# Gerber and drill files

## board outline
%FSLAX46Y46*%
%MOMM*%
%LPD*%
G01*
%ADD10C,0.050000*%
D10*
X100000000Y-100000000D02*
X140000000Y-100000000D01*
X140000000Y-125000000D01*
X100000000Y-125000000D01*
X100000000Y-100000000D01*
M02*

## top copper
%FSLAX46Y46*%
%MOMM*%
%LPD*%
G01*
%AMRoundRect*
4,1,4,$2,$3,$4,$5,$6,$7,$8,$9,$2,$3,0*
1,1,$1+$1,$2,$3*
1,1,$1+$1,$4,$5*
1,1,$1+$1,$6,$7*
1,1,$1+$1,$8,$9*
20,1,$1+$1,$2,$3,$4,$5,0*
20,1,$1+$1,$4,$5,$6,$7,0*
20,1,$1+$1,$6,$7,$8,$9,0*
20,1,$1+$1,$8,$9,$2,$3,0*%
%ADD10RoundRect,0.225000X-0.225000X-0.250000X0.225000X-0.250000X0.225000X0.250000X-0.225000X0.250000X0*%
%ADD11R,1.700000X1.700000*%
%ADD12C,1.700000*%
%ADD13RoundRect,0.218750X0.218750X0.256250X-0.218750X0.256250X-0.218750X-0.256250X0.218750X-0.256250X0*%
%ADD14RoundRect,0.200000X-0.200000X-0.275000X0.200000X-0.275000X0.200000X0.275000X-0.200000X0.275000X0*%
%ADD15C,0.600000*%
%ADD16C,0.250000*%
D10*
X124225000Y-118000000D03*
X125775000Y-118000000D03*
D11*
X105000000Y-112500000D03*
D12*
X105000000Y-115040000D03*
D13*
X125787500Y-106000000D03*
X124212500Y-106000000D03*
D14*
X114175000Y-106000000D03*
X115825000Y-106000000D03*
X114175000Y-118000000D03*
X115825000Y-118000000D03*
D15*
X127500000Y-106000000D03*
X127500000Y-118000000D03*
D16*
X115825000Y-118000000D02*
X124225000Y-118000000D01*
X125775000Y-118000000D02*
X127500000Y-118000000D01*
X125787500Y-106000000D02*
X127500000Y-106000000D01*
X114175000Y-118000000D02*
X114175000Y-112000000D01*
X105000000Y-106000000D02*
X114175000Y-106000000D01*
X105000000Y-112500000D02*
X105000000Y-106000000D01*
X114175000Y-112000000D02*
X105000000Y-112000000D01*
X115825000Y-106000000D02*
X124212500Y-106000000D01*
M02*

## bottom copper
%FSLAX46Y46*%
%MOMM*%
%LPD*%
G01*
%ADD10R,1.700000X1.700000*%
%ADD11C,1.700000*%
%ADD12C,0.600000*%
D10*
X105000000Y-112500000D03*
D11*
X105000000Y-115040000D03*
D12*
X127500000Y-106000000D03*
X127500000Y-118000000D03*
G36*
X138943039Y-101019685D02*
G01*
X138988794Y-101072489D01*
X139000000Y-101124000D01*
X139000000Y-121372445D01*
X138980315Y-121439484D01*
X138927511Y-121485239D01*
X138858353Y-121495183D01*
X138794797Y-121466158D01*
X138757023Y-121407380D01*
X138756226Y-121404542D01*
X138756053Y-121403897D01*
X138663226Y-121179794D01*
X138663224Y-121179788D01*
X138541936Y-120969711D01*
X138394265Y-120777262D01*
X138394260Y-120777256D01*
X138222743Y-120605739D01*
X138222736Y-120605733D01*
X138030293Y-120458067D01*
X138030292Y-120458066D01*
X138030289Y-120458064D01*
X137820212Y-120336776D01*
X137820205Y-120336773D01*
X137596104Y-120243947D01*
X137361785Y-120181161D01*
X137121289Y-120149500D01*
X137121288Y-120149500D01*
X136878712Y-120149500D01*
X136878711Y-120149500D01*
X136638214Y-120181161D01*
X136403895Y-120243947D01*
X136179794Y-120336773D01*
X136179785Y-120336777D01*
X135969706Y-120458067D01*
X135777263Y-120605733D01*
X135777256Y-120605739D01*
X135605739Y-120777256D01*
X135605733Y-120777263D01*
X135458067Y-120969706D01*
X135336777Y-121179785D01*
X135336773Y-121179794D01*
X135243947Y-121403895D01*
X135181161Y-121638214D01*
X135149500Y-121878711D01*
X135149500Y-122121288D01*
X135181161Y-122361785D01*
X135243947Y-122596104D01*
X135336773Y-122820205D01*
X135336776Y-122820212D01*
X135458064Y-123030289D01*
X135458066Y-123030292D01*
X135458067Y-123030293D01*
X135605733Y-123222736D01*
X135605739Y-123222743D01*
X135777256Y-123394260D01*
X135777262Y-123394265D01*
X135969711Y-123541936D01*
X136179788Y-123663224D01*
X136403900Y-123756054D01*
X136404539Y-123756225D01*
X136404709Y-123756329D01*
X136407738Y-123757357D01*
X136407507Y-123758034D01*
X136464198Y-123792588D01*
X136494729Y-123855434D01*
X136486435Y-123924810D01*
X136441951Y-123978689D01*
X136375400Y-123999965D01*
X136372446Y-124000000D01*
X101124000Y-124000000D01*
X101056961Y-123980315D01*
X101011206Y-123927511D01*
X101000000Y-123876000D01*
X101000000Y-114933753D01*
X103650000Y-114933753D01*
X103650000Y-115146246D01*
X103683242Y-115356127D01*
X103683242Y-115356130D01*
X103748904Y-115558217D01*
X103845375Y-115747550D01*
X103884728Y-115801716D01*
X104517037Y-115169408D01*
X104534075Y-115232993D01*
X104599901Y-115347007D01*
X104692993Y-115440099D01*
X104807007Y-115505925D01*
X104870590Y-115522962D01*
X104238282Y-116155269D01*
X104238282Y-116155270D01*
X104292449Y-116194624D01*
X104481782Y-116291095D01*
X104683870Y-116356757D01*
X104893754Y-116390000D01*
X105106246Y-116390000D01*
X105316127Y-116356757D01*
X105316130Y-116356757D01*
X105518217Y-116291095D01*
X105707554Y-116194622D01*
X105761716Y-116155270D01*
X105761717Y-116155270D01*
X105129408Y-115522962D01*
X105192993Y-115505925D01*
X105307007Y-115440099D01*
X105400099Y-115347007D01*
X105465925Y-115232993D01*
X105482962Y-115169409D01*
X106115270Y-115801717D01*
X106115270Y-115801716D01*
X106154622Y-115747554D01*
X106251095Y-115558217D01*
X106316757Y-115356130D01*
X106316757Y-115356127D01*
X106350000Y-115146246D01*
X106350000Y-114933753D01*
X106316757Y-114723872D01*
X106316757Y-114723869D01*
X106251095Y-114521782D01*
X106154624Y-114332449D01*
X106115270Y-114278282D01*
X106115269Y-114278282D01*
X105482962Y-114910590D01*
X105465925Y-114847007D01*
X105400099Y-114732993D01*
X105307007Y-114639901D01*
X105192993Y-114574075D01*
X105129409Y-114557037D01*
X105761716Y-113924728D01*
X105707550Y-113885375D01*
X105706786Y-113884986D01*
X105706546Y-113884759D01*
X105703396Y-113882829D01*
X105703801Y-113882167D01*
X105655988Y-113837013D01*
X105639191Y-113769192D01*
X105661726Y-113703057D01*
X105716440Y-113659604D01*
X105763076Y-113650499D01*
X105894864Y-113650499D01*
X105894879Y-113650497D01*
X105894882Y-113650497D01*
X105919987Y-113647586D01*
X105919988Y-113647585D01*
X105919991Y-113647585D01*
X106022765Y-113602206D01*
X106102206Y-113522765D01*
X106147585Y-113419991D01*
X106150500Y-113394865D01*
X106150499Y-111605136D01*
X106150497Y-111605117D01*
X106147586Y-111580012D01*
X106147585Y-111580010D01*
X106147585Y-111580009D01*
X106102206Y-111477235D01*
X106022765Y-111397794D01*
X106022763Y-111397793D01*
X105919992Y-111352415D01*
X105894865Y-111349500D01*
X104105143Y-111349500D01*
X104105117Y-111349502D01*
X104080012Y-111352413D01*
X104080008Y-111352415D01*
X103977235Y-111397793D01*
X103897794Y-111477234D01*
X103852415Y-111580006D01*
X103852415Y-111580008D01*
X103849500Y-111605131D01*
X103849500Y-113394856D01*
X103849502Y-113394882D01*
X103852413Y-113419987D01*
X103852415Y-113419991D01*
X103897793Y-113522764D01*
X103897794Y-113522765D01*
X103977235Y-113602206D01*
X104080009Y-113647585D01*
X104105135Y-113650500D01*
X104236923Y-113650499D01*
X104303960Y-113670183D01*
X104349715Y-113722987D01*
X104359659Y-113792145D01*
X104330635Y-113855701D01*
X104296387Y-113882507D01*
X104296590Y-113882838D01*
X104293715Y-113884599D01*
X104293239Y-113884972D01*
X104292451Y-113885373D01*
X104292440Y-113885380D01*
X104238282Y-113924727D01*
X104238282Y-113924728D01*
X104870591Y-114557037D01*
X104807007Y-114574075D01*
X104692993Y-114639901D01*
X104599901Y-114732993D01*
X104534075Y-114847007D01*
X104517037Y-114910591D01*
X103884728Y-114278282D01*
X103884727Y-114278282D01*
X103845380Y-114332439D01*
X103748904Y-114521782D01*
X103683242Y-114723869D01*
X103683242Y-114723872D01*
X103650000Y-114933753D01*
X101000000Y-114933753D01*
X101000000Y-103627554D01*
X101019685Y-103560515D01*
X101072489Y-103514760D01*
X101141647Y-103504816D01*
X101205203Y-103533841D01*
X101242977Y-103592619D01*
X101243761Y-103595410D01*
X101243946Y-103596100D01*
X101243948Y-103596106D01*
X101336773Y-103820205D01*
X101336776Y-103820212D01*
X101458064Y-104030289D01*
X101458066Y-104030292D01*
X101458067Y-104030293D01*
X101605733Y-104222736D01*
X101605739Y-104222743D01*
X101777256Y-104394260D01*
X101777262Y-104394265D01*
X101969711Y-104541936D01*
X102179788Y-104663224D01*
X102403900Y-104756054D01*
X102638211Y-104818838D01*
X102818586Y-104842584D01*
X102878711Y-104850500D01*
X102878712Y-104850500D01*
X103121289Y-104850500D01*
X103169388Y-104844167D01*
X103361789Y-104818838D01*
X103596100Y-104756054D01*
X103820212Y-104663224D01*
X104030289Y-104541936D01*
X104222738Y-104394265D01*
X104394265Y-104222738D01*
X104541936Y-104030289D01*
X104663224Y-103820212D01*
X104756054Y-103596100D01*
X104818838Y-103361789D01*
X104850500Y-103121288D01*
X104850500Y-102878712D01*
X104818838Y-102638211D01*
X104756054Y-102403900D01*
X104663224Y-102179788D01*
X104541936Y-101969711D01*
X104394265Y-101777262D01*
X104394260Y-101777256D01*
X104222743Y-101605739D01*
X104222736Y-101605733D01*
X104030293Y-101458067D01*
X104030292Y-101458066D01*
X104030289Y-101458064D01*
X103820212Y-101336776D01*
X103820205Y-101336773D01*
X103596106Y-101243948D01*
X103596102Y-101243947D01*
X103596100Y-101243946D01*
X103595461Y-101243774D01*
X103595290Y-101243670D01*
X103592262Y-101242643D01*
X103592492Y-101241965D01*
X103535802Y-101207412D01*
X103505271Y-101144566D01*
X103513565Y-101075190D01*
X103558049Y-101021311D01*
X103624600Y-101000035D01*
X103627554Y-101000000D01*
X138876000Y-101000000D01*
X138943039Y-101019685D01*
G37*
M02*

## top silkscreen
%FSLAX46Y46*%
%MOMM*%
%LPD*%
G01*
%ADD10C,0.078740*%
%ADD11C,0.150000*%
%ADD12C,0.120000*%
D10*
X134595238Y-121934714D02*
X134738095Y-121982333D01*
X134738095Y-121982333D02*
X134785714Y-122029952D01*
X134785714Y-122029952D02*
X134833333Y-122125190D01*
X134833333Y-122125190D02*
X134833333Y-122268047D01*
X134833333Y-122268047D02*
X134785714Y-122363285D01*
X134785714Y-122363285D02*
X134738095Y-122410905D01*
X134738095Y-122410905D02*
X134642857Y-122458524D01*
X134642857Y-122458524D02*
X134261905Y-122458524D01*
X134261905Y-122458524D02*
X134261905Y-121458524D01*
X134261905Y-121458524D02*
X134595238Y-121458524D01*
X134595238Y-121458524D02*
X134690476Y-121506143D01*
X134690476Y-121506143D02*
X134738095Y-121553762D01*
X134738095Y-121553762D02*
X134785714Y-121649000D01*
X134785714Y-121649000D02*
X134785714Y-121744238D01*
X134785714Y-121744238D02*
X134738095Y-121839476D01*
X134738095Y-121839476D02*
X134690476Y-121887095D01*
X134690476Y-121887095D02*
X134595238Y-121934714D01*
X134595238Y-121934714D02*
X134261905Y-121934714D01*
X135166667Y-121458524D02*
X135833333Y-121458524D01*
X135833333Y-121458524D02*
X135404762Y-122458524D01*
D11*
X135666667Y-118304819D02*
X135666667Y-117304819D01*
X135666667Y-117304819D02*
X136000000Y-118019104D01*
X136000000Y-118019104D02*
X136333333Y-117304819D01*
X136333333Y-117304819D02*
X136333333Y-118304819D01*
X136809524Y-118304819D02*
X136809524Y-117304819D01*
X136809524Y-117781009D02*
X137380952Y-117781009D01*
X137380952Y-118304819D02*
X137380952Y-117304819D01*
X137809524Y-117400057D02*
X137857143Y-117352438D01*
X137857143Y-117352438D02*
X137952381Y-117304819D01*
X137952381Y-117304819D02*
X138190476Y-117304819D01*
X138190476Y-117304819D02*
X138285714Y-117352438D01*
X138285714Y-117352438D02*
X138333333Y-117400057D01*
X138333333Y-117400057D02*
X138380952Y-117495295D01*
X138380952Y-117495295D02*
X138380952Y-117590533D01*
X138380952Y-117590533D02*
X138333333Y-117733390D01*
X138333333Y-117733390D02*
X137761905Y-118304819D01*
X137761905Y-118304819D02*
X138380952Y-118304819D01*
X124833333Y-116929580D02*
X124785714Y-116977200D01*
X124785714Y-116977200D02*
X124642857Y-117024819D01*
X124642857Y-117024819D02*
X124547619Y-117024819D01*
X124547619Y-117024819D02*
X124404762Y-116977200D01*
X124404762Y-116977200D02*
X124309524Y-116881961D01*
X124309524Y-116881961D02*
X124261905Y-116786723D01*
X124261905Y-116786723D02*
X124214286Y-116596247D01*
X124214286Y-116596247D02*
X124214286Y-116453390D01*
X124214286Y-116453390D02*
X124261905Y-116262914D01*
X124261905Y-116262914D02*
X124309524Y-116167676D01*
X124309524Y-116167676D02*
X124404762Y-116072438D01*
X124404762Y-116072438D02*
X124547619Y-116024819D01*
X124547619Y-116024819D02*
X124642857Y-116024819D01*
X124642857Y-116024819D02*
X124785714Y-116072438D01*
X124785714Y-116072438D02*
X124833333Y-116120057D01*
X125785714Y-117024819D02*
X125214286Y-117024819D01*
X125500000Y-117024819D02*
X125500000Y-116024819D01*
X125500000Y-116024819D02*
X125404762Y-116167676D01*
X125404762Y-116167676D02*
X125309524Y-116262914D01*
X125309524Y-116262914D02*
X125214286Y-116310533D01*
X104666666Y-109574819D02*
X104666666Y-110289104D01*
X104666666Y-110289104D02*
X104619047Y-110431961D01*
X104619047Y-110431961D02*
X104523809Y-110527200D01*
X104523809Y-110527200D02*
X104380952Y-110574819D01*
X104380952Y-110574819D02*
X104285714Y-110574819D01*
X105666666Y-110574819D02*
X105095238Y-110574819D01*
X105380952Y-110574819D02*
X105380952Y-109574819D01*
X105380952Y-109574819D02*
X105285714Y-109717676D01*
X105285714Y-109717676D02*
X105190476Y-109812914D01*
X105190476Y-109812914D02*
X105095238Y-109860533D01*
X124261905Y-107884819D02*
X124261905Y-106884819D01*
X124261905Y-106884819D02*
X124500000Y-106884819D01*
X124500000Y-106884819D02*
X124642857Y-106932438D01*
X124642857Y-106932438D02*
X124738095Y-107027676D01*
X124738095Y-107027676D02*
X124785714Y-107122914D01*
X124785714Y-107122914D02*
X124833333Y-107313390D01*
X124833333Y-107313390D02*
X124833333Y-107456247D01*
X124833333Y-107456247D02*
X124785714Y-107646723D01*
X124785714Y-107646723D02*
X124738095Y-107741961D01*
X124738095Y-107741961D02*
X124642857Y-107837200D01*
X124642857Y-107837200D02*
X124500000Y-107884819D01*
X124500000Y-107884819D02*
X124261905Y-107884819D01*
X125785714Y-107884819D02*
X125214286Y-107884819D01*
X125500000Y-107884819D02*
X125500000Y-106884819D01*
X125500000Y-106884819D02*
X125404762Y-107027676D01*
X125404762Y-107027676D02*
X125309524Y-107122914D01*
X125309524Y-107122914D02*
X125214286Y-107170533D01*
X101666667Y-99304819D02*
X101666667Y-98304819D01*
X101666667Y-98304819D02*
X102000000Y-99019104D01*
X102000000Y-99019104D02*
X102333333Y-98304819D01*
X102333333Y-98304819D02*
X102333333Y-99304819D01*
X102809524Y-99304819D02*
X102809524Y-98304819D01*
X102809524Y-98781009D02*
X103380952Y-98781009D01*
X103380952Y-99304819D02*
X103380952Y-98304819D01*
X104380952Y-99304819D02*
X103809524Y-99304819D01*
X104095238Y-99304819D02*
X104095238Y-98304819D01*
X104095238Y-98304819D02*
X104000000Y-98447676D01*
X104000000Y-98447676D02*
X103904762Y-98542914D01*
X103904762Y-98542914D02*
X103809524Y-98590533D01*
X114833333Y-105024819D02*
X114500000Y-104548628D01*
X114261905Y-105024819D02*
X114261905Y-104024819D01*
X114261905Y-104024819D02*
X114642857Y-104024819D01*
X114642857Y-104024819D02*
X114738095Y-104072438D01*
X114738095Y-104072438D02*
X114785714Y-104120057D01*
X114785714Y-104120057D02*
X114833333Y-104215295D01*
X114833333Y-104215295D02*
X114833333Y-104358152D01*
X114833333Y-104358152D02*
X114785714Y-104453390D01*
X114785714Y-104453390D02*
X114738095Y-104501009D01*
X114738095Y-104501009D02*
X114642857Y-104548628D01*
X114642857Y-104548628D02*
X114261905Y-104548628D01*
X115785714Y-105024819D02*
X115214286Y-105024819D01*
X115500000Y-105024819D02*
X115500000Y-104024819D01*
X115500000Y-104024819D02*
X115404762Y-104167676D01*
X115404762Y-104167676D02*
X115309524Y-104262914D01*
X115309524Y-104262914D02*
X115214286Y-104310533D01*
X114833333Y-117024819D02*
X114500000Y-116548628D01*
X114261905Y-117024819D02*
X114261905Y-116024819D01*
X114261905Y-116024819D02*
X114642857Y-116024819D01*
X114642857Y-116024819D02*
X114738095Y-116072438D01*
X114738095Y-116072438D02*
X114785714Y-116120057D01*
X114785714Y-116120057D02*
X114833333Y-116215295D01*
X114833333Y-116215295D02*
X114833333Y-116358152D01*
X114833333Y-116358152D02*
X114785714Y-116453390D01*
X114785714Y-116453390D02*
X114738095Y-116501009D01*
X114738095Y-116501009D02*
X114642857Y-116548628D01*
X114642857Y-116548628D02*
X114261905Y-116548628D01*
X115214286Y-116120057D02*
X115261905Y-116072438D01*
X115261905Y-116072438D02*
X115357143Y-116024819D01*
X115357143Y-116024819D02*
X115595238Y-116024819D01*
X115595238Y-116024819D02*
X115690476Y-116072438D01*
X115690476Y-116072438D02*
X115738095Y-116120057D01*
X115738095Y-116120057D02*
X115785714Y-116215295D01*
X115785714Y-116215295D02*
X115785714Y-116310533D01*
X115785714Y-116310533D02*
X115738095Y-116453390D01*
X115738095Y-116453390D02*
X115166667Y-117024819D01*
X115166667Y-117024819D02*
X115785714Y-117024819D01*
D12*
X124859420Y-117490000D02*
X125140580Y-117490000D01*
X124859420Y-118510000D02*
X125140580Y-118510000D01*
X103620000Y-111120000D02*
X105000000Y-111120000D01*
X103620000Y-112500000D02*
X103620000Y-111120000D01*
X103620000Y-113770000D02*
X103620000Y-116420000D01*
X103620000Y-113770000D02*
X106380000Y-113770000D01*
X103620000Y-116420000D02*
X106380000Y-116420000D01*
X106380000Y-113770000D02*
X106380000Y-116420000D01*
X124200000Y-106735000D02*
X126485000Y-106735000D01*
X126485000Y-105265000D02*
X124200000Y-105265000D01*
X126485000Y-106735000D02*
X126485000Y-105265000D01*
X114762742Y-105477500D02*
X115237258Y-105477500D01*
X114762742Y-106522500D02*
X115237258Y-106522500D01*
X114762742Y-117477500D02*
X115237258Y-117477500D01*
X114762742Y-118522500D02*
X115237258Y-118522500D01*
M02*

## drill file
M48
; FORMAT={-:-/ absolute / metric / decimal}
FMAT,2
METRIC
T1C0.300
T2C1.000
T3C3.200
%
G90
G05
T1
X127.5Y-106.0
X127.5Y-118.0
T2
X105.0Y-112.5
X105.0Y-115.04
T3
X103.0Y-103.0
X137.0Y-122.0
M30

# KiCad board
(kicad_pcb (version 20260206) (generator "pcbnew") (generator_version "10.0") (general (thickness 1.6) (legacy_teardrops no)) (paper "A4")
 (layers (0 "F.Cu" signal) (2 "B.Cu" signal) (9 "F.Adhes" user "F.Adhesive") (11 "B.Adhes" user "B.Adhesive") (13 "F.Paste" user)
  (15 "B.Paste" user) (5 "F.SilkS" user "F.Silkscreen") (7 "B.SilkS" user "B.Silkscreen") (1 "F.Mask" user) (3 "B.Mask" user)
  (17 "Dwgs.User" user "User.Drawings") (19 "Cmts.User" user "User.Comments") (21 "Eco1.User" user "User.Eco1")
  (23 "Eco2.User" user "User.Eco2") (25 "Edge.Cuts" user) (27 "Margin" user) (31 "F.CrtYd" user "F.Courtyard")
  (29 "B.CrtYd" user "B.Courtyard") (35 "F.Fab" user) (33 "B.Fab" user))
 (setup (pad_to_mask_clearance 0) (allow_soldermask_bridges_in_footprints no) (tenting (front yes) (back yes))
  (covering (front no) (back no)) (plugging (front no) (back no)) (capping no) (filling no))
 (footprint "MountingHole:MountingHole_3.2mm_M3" (layer "F.Cu") (at 137 122)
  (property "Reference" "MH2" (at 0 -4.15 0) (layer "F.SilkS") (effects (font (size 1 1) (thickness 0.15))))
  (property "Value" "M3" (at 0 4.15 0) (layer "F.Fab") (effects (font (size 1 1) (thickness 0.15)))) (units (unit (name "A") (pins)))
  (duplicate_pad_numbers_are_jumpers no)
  (pad "" np_thru_hole circle (at 0 0) (size 3.2 3.2) (drill 3.2) (layers "*.Cu" "*.Mask")))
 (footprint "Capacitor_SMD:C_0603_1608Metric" (layer "F.Cu") (at 125 118)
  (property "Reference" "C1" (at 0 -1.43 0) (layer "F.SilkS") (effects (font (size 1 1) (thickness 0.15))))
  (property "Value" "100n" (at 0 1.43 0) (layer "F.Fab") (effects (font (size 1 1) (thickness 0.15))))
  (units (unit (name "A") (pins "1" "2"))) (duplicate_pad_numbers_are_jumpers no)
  (fp_line (start -0.14058 -0.51) (end 0.14058 -0.51) (stroke (width 0.12) (type solid)) (layer "F.SilkS"))
  (fp_line (start -0.14058 0.51) (end 0.14058 0.51) (stroke (width 0.12) (type solid)) (layer "F.SilkS"))
  (pad "1" smd roundrect (at -0.775 0) (size 0.9 0.95) (layers "F.Cu" "F.Mask" "F.Paste") (roundrect_rratio 0.25) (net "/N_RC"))
  (pad "2" smd roundrect (at 0.775 0) (size 0.9 0.95) (layers "F.Cu" "F.Mask" "F.Paste") (roundrect_rratio 0.25) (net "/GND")))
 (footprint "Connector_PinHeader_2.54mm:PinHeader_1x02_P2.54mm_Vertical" (layer "F.Cu") (at 105 112.5)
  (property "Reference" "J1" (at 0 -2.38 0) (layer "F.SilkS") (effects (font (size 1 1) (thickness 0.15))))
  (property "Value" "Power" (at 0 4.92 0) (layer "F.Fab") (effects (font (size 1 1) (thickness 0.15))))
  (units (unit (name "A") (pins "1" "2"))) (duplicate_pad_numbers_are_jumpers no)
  (fp_line (start -1.38 -1.38) (end 0 -1.38) (stroke (width 0.12) (type solid)) (layer "F.SilkS"))
  (fp_line (start -1.38 0) (end -1.38 -1.38) (stroke (width 0.12) (type solid)) (layer "F.SilkS"))
  (fp_line (start -1.38 1.27) (end -1.38 3.92) (stroke (width 0.12) (type solid)) (layer "F.SilkS"))
  (fp_line (start -1.38 1.27) (end 1.38 1.27) (stroke (width 0.12) (type solid)) (layer "F.SilkS"))
  (fp_line (start -1.38 3.92) (end 1.38 3.92) (stroke (width 0.12) (type solid)) (layer "F.SilkS"))
  (fp_line (start 1.38 1.27) (end 1.38 3.92) (stroke (width 0.12) (type solid)) (layer "F.SilkS"))
  (pad "1" thru_hole rect (at 0 0) (size 1.7 1.7) (drill 1) (layers "*.Cu" "*.Mask") (remove_unused_layers no) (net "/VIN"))
  (pad "2" thru_hole circle (at 0 2.54) (size 1.7 1.7) (drill 1) (layers "*.Cu" "*.Mask") (remove_unused_layers no) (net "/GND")))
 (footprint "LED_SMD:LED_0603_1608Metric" (layer "F.Cu") (at 125 106 180)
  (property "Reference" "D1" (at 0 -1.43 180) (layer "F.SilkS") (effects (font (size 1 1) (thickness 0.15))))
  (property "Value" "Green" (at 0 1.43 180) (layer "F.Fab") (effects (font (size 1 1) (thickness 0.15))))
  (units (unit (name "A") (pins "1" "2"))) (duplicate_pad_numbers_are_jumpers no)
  (fp_line (start 0.8 -0.735) (end -1.485 -0.735) (stroke (width 0.12) (type solid)) (layer "F.SilkS"))
  (fp_line (start -1.485 0.735) (end 0.8 0.735) (stroke (width 0.12) (type solid)) (layer "F.SilkS"))
  (fp_line (start -1.485 -0.735) (end -1.485 0.735) (stroke (width 0.12) (type solid)) (layer "F.SilkS"))
  (pad "1" smd roundrect (at -0.7875 0 180) (size 0.875 0.95) (layers "F.Cu" "F.Mask" "F.Paste") (roundrect_rratio 0.25) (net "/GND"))
  (pad "2" smd roundrect (at 0.7875 0 180) (size 0.875 0.95) (layers "F.Cu" "F.Mask" "F.Paste") (roundrect_rratio 0.25) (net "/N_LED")))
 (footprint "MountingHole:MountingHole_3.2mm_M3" (layer "F.Cu") (at 103 103)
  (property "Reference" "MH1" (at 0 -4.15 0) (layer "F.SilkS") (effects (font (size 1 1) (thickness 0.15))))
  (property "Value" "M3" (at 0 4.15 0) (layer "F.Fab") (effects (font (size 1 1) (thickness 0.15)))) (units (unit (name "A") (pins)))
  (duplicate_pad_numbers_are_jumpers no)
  (pad "" np_thru_hole circle (at 0 0) (size 3.2 3.2) (drill 3.2) (layers "*.Cu" "*.Mask")))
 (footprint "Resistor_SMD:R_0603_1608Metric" (layer "F.Cu") (at 115 106)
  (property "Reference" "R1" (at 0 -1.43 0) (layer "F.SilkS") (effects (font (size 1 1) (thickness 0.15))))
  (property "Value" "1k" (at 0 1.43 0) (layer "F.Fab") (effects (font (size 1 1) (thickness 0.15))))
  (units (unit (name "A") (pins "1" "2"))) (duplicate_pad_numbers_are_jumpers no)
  (fp_line (start -0.237258 -0.5225) (end 0.237258 -0.5225) (stroke (width 0.12) (type solid)) (layer "F.SilkS"))
  (fp_line (start -0.237258 0.5225) (end 0.237258 0.5225) (stroke (width 0.12) (type solid)) (layer "F.SilkS"))
  (pad "1" smd roundrect (at -0.825 0) (size 0.8 0.95) (layers "F.Cu" "F.Mask" "F.Paste") (roundrect_rratio 0.25) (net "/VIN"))
  (pad "2" smd roundrect (at 0.825 0) (size 0.8 0.95) (layers "F.Cu" "F.Mask" "F.Paste") (roundrect_rratio 0.25) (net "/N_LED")))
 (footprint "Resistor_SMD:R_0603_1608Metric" (layer "F.Cu") (at 115 118)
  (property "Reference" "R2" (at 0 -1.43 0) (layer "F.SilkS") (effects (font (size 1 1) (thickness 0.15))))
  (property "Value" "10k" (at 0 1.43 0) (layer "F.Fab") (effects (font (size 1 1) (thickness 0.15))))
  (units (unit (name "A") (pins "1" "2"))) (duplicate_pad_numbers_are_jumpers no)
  (fp_line (start -0.237258 -0.5225) (end 0.237258 -0.5225) (stroke (width 0.12) (type solid)) (layer "F.SilkS"))
  (fp_line (start -0.237258 0.5225) (end 0.237258 0.5225) (stroke (width 0.12) (type solid)) (layer "F.SilkS"))
  (pad "1" smd roundrect (at -0.825 0) (size 0.8 0.95) (layers "F.Cu" "F.Mask" "F.Paste") (roundrect_rratio 0.25) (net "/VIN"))
  (pad "2" smd roundrect (at 0.825 0) (size 0.8 0.95) (layers "F.Cu" "F.Mask" "F.Paste") (roundrect_rratio 0.25) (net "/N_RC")))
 (gr_rect (start 100 100) (end 140 125) (stroke (width 0.05) (type default)) (fill no) (layer "Edge.Cuts"))
 (segment (start 115.825 118) (end 124.225 118) (width 0.25) (layer "F.Cu") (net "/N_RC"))
 (segment (start 125.775 118) (end 127.5 118) (width 0.25) (layer "F.Cu") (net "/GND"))
 (segment (start 125.7875 106) (end 127.5 106) (width 0.25) (layer "F.Cu") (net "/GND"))
 (via (at 127.5 106) (size 0.6) (drill 0.3) (layers "F.Cu" "B.Cu") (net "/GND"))
 (via (at 127.5 118) (size 0.6) (drill 0.3) (layers "F.Cu" "B.Cu") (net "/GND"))
 (segment (start 114.175 118) (end 114.175 112) (width 0.25) (layer "F.Cu") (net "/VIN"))
 (segment (start 105 106) (end 114.175 106) (width 0.25) (layer "F.Cu") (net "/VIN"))
 (segment (start 105 112.5) (end 105 106) (width 0.25) (layer "F.Cu") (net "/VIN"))
 (segment (start 114.175 112) (end 105 112) (width 0.25) (layer "F.Cu") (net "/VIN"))
 (segment (start 115.825 106) (end 124.2125 106) (width 0.25) (layer "F.Cu") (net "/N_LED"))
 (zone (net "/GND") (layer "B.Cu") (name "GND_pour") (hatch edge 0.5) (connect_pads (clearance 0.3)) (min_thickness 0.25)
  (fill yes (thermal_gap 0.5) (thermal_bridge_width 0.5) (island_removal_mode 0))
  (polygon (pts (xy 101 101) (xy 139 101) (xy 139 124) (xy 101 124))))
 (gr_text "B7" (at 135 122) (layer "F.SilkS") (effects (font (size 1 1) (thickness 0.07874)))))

